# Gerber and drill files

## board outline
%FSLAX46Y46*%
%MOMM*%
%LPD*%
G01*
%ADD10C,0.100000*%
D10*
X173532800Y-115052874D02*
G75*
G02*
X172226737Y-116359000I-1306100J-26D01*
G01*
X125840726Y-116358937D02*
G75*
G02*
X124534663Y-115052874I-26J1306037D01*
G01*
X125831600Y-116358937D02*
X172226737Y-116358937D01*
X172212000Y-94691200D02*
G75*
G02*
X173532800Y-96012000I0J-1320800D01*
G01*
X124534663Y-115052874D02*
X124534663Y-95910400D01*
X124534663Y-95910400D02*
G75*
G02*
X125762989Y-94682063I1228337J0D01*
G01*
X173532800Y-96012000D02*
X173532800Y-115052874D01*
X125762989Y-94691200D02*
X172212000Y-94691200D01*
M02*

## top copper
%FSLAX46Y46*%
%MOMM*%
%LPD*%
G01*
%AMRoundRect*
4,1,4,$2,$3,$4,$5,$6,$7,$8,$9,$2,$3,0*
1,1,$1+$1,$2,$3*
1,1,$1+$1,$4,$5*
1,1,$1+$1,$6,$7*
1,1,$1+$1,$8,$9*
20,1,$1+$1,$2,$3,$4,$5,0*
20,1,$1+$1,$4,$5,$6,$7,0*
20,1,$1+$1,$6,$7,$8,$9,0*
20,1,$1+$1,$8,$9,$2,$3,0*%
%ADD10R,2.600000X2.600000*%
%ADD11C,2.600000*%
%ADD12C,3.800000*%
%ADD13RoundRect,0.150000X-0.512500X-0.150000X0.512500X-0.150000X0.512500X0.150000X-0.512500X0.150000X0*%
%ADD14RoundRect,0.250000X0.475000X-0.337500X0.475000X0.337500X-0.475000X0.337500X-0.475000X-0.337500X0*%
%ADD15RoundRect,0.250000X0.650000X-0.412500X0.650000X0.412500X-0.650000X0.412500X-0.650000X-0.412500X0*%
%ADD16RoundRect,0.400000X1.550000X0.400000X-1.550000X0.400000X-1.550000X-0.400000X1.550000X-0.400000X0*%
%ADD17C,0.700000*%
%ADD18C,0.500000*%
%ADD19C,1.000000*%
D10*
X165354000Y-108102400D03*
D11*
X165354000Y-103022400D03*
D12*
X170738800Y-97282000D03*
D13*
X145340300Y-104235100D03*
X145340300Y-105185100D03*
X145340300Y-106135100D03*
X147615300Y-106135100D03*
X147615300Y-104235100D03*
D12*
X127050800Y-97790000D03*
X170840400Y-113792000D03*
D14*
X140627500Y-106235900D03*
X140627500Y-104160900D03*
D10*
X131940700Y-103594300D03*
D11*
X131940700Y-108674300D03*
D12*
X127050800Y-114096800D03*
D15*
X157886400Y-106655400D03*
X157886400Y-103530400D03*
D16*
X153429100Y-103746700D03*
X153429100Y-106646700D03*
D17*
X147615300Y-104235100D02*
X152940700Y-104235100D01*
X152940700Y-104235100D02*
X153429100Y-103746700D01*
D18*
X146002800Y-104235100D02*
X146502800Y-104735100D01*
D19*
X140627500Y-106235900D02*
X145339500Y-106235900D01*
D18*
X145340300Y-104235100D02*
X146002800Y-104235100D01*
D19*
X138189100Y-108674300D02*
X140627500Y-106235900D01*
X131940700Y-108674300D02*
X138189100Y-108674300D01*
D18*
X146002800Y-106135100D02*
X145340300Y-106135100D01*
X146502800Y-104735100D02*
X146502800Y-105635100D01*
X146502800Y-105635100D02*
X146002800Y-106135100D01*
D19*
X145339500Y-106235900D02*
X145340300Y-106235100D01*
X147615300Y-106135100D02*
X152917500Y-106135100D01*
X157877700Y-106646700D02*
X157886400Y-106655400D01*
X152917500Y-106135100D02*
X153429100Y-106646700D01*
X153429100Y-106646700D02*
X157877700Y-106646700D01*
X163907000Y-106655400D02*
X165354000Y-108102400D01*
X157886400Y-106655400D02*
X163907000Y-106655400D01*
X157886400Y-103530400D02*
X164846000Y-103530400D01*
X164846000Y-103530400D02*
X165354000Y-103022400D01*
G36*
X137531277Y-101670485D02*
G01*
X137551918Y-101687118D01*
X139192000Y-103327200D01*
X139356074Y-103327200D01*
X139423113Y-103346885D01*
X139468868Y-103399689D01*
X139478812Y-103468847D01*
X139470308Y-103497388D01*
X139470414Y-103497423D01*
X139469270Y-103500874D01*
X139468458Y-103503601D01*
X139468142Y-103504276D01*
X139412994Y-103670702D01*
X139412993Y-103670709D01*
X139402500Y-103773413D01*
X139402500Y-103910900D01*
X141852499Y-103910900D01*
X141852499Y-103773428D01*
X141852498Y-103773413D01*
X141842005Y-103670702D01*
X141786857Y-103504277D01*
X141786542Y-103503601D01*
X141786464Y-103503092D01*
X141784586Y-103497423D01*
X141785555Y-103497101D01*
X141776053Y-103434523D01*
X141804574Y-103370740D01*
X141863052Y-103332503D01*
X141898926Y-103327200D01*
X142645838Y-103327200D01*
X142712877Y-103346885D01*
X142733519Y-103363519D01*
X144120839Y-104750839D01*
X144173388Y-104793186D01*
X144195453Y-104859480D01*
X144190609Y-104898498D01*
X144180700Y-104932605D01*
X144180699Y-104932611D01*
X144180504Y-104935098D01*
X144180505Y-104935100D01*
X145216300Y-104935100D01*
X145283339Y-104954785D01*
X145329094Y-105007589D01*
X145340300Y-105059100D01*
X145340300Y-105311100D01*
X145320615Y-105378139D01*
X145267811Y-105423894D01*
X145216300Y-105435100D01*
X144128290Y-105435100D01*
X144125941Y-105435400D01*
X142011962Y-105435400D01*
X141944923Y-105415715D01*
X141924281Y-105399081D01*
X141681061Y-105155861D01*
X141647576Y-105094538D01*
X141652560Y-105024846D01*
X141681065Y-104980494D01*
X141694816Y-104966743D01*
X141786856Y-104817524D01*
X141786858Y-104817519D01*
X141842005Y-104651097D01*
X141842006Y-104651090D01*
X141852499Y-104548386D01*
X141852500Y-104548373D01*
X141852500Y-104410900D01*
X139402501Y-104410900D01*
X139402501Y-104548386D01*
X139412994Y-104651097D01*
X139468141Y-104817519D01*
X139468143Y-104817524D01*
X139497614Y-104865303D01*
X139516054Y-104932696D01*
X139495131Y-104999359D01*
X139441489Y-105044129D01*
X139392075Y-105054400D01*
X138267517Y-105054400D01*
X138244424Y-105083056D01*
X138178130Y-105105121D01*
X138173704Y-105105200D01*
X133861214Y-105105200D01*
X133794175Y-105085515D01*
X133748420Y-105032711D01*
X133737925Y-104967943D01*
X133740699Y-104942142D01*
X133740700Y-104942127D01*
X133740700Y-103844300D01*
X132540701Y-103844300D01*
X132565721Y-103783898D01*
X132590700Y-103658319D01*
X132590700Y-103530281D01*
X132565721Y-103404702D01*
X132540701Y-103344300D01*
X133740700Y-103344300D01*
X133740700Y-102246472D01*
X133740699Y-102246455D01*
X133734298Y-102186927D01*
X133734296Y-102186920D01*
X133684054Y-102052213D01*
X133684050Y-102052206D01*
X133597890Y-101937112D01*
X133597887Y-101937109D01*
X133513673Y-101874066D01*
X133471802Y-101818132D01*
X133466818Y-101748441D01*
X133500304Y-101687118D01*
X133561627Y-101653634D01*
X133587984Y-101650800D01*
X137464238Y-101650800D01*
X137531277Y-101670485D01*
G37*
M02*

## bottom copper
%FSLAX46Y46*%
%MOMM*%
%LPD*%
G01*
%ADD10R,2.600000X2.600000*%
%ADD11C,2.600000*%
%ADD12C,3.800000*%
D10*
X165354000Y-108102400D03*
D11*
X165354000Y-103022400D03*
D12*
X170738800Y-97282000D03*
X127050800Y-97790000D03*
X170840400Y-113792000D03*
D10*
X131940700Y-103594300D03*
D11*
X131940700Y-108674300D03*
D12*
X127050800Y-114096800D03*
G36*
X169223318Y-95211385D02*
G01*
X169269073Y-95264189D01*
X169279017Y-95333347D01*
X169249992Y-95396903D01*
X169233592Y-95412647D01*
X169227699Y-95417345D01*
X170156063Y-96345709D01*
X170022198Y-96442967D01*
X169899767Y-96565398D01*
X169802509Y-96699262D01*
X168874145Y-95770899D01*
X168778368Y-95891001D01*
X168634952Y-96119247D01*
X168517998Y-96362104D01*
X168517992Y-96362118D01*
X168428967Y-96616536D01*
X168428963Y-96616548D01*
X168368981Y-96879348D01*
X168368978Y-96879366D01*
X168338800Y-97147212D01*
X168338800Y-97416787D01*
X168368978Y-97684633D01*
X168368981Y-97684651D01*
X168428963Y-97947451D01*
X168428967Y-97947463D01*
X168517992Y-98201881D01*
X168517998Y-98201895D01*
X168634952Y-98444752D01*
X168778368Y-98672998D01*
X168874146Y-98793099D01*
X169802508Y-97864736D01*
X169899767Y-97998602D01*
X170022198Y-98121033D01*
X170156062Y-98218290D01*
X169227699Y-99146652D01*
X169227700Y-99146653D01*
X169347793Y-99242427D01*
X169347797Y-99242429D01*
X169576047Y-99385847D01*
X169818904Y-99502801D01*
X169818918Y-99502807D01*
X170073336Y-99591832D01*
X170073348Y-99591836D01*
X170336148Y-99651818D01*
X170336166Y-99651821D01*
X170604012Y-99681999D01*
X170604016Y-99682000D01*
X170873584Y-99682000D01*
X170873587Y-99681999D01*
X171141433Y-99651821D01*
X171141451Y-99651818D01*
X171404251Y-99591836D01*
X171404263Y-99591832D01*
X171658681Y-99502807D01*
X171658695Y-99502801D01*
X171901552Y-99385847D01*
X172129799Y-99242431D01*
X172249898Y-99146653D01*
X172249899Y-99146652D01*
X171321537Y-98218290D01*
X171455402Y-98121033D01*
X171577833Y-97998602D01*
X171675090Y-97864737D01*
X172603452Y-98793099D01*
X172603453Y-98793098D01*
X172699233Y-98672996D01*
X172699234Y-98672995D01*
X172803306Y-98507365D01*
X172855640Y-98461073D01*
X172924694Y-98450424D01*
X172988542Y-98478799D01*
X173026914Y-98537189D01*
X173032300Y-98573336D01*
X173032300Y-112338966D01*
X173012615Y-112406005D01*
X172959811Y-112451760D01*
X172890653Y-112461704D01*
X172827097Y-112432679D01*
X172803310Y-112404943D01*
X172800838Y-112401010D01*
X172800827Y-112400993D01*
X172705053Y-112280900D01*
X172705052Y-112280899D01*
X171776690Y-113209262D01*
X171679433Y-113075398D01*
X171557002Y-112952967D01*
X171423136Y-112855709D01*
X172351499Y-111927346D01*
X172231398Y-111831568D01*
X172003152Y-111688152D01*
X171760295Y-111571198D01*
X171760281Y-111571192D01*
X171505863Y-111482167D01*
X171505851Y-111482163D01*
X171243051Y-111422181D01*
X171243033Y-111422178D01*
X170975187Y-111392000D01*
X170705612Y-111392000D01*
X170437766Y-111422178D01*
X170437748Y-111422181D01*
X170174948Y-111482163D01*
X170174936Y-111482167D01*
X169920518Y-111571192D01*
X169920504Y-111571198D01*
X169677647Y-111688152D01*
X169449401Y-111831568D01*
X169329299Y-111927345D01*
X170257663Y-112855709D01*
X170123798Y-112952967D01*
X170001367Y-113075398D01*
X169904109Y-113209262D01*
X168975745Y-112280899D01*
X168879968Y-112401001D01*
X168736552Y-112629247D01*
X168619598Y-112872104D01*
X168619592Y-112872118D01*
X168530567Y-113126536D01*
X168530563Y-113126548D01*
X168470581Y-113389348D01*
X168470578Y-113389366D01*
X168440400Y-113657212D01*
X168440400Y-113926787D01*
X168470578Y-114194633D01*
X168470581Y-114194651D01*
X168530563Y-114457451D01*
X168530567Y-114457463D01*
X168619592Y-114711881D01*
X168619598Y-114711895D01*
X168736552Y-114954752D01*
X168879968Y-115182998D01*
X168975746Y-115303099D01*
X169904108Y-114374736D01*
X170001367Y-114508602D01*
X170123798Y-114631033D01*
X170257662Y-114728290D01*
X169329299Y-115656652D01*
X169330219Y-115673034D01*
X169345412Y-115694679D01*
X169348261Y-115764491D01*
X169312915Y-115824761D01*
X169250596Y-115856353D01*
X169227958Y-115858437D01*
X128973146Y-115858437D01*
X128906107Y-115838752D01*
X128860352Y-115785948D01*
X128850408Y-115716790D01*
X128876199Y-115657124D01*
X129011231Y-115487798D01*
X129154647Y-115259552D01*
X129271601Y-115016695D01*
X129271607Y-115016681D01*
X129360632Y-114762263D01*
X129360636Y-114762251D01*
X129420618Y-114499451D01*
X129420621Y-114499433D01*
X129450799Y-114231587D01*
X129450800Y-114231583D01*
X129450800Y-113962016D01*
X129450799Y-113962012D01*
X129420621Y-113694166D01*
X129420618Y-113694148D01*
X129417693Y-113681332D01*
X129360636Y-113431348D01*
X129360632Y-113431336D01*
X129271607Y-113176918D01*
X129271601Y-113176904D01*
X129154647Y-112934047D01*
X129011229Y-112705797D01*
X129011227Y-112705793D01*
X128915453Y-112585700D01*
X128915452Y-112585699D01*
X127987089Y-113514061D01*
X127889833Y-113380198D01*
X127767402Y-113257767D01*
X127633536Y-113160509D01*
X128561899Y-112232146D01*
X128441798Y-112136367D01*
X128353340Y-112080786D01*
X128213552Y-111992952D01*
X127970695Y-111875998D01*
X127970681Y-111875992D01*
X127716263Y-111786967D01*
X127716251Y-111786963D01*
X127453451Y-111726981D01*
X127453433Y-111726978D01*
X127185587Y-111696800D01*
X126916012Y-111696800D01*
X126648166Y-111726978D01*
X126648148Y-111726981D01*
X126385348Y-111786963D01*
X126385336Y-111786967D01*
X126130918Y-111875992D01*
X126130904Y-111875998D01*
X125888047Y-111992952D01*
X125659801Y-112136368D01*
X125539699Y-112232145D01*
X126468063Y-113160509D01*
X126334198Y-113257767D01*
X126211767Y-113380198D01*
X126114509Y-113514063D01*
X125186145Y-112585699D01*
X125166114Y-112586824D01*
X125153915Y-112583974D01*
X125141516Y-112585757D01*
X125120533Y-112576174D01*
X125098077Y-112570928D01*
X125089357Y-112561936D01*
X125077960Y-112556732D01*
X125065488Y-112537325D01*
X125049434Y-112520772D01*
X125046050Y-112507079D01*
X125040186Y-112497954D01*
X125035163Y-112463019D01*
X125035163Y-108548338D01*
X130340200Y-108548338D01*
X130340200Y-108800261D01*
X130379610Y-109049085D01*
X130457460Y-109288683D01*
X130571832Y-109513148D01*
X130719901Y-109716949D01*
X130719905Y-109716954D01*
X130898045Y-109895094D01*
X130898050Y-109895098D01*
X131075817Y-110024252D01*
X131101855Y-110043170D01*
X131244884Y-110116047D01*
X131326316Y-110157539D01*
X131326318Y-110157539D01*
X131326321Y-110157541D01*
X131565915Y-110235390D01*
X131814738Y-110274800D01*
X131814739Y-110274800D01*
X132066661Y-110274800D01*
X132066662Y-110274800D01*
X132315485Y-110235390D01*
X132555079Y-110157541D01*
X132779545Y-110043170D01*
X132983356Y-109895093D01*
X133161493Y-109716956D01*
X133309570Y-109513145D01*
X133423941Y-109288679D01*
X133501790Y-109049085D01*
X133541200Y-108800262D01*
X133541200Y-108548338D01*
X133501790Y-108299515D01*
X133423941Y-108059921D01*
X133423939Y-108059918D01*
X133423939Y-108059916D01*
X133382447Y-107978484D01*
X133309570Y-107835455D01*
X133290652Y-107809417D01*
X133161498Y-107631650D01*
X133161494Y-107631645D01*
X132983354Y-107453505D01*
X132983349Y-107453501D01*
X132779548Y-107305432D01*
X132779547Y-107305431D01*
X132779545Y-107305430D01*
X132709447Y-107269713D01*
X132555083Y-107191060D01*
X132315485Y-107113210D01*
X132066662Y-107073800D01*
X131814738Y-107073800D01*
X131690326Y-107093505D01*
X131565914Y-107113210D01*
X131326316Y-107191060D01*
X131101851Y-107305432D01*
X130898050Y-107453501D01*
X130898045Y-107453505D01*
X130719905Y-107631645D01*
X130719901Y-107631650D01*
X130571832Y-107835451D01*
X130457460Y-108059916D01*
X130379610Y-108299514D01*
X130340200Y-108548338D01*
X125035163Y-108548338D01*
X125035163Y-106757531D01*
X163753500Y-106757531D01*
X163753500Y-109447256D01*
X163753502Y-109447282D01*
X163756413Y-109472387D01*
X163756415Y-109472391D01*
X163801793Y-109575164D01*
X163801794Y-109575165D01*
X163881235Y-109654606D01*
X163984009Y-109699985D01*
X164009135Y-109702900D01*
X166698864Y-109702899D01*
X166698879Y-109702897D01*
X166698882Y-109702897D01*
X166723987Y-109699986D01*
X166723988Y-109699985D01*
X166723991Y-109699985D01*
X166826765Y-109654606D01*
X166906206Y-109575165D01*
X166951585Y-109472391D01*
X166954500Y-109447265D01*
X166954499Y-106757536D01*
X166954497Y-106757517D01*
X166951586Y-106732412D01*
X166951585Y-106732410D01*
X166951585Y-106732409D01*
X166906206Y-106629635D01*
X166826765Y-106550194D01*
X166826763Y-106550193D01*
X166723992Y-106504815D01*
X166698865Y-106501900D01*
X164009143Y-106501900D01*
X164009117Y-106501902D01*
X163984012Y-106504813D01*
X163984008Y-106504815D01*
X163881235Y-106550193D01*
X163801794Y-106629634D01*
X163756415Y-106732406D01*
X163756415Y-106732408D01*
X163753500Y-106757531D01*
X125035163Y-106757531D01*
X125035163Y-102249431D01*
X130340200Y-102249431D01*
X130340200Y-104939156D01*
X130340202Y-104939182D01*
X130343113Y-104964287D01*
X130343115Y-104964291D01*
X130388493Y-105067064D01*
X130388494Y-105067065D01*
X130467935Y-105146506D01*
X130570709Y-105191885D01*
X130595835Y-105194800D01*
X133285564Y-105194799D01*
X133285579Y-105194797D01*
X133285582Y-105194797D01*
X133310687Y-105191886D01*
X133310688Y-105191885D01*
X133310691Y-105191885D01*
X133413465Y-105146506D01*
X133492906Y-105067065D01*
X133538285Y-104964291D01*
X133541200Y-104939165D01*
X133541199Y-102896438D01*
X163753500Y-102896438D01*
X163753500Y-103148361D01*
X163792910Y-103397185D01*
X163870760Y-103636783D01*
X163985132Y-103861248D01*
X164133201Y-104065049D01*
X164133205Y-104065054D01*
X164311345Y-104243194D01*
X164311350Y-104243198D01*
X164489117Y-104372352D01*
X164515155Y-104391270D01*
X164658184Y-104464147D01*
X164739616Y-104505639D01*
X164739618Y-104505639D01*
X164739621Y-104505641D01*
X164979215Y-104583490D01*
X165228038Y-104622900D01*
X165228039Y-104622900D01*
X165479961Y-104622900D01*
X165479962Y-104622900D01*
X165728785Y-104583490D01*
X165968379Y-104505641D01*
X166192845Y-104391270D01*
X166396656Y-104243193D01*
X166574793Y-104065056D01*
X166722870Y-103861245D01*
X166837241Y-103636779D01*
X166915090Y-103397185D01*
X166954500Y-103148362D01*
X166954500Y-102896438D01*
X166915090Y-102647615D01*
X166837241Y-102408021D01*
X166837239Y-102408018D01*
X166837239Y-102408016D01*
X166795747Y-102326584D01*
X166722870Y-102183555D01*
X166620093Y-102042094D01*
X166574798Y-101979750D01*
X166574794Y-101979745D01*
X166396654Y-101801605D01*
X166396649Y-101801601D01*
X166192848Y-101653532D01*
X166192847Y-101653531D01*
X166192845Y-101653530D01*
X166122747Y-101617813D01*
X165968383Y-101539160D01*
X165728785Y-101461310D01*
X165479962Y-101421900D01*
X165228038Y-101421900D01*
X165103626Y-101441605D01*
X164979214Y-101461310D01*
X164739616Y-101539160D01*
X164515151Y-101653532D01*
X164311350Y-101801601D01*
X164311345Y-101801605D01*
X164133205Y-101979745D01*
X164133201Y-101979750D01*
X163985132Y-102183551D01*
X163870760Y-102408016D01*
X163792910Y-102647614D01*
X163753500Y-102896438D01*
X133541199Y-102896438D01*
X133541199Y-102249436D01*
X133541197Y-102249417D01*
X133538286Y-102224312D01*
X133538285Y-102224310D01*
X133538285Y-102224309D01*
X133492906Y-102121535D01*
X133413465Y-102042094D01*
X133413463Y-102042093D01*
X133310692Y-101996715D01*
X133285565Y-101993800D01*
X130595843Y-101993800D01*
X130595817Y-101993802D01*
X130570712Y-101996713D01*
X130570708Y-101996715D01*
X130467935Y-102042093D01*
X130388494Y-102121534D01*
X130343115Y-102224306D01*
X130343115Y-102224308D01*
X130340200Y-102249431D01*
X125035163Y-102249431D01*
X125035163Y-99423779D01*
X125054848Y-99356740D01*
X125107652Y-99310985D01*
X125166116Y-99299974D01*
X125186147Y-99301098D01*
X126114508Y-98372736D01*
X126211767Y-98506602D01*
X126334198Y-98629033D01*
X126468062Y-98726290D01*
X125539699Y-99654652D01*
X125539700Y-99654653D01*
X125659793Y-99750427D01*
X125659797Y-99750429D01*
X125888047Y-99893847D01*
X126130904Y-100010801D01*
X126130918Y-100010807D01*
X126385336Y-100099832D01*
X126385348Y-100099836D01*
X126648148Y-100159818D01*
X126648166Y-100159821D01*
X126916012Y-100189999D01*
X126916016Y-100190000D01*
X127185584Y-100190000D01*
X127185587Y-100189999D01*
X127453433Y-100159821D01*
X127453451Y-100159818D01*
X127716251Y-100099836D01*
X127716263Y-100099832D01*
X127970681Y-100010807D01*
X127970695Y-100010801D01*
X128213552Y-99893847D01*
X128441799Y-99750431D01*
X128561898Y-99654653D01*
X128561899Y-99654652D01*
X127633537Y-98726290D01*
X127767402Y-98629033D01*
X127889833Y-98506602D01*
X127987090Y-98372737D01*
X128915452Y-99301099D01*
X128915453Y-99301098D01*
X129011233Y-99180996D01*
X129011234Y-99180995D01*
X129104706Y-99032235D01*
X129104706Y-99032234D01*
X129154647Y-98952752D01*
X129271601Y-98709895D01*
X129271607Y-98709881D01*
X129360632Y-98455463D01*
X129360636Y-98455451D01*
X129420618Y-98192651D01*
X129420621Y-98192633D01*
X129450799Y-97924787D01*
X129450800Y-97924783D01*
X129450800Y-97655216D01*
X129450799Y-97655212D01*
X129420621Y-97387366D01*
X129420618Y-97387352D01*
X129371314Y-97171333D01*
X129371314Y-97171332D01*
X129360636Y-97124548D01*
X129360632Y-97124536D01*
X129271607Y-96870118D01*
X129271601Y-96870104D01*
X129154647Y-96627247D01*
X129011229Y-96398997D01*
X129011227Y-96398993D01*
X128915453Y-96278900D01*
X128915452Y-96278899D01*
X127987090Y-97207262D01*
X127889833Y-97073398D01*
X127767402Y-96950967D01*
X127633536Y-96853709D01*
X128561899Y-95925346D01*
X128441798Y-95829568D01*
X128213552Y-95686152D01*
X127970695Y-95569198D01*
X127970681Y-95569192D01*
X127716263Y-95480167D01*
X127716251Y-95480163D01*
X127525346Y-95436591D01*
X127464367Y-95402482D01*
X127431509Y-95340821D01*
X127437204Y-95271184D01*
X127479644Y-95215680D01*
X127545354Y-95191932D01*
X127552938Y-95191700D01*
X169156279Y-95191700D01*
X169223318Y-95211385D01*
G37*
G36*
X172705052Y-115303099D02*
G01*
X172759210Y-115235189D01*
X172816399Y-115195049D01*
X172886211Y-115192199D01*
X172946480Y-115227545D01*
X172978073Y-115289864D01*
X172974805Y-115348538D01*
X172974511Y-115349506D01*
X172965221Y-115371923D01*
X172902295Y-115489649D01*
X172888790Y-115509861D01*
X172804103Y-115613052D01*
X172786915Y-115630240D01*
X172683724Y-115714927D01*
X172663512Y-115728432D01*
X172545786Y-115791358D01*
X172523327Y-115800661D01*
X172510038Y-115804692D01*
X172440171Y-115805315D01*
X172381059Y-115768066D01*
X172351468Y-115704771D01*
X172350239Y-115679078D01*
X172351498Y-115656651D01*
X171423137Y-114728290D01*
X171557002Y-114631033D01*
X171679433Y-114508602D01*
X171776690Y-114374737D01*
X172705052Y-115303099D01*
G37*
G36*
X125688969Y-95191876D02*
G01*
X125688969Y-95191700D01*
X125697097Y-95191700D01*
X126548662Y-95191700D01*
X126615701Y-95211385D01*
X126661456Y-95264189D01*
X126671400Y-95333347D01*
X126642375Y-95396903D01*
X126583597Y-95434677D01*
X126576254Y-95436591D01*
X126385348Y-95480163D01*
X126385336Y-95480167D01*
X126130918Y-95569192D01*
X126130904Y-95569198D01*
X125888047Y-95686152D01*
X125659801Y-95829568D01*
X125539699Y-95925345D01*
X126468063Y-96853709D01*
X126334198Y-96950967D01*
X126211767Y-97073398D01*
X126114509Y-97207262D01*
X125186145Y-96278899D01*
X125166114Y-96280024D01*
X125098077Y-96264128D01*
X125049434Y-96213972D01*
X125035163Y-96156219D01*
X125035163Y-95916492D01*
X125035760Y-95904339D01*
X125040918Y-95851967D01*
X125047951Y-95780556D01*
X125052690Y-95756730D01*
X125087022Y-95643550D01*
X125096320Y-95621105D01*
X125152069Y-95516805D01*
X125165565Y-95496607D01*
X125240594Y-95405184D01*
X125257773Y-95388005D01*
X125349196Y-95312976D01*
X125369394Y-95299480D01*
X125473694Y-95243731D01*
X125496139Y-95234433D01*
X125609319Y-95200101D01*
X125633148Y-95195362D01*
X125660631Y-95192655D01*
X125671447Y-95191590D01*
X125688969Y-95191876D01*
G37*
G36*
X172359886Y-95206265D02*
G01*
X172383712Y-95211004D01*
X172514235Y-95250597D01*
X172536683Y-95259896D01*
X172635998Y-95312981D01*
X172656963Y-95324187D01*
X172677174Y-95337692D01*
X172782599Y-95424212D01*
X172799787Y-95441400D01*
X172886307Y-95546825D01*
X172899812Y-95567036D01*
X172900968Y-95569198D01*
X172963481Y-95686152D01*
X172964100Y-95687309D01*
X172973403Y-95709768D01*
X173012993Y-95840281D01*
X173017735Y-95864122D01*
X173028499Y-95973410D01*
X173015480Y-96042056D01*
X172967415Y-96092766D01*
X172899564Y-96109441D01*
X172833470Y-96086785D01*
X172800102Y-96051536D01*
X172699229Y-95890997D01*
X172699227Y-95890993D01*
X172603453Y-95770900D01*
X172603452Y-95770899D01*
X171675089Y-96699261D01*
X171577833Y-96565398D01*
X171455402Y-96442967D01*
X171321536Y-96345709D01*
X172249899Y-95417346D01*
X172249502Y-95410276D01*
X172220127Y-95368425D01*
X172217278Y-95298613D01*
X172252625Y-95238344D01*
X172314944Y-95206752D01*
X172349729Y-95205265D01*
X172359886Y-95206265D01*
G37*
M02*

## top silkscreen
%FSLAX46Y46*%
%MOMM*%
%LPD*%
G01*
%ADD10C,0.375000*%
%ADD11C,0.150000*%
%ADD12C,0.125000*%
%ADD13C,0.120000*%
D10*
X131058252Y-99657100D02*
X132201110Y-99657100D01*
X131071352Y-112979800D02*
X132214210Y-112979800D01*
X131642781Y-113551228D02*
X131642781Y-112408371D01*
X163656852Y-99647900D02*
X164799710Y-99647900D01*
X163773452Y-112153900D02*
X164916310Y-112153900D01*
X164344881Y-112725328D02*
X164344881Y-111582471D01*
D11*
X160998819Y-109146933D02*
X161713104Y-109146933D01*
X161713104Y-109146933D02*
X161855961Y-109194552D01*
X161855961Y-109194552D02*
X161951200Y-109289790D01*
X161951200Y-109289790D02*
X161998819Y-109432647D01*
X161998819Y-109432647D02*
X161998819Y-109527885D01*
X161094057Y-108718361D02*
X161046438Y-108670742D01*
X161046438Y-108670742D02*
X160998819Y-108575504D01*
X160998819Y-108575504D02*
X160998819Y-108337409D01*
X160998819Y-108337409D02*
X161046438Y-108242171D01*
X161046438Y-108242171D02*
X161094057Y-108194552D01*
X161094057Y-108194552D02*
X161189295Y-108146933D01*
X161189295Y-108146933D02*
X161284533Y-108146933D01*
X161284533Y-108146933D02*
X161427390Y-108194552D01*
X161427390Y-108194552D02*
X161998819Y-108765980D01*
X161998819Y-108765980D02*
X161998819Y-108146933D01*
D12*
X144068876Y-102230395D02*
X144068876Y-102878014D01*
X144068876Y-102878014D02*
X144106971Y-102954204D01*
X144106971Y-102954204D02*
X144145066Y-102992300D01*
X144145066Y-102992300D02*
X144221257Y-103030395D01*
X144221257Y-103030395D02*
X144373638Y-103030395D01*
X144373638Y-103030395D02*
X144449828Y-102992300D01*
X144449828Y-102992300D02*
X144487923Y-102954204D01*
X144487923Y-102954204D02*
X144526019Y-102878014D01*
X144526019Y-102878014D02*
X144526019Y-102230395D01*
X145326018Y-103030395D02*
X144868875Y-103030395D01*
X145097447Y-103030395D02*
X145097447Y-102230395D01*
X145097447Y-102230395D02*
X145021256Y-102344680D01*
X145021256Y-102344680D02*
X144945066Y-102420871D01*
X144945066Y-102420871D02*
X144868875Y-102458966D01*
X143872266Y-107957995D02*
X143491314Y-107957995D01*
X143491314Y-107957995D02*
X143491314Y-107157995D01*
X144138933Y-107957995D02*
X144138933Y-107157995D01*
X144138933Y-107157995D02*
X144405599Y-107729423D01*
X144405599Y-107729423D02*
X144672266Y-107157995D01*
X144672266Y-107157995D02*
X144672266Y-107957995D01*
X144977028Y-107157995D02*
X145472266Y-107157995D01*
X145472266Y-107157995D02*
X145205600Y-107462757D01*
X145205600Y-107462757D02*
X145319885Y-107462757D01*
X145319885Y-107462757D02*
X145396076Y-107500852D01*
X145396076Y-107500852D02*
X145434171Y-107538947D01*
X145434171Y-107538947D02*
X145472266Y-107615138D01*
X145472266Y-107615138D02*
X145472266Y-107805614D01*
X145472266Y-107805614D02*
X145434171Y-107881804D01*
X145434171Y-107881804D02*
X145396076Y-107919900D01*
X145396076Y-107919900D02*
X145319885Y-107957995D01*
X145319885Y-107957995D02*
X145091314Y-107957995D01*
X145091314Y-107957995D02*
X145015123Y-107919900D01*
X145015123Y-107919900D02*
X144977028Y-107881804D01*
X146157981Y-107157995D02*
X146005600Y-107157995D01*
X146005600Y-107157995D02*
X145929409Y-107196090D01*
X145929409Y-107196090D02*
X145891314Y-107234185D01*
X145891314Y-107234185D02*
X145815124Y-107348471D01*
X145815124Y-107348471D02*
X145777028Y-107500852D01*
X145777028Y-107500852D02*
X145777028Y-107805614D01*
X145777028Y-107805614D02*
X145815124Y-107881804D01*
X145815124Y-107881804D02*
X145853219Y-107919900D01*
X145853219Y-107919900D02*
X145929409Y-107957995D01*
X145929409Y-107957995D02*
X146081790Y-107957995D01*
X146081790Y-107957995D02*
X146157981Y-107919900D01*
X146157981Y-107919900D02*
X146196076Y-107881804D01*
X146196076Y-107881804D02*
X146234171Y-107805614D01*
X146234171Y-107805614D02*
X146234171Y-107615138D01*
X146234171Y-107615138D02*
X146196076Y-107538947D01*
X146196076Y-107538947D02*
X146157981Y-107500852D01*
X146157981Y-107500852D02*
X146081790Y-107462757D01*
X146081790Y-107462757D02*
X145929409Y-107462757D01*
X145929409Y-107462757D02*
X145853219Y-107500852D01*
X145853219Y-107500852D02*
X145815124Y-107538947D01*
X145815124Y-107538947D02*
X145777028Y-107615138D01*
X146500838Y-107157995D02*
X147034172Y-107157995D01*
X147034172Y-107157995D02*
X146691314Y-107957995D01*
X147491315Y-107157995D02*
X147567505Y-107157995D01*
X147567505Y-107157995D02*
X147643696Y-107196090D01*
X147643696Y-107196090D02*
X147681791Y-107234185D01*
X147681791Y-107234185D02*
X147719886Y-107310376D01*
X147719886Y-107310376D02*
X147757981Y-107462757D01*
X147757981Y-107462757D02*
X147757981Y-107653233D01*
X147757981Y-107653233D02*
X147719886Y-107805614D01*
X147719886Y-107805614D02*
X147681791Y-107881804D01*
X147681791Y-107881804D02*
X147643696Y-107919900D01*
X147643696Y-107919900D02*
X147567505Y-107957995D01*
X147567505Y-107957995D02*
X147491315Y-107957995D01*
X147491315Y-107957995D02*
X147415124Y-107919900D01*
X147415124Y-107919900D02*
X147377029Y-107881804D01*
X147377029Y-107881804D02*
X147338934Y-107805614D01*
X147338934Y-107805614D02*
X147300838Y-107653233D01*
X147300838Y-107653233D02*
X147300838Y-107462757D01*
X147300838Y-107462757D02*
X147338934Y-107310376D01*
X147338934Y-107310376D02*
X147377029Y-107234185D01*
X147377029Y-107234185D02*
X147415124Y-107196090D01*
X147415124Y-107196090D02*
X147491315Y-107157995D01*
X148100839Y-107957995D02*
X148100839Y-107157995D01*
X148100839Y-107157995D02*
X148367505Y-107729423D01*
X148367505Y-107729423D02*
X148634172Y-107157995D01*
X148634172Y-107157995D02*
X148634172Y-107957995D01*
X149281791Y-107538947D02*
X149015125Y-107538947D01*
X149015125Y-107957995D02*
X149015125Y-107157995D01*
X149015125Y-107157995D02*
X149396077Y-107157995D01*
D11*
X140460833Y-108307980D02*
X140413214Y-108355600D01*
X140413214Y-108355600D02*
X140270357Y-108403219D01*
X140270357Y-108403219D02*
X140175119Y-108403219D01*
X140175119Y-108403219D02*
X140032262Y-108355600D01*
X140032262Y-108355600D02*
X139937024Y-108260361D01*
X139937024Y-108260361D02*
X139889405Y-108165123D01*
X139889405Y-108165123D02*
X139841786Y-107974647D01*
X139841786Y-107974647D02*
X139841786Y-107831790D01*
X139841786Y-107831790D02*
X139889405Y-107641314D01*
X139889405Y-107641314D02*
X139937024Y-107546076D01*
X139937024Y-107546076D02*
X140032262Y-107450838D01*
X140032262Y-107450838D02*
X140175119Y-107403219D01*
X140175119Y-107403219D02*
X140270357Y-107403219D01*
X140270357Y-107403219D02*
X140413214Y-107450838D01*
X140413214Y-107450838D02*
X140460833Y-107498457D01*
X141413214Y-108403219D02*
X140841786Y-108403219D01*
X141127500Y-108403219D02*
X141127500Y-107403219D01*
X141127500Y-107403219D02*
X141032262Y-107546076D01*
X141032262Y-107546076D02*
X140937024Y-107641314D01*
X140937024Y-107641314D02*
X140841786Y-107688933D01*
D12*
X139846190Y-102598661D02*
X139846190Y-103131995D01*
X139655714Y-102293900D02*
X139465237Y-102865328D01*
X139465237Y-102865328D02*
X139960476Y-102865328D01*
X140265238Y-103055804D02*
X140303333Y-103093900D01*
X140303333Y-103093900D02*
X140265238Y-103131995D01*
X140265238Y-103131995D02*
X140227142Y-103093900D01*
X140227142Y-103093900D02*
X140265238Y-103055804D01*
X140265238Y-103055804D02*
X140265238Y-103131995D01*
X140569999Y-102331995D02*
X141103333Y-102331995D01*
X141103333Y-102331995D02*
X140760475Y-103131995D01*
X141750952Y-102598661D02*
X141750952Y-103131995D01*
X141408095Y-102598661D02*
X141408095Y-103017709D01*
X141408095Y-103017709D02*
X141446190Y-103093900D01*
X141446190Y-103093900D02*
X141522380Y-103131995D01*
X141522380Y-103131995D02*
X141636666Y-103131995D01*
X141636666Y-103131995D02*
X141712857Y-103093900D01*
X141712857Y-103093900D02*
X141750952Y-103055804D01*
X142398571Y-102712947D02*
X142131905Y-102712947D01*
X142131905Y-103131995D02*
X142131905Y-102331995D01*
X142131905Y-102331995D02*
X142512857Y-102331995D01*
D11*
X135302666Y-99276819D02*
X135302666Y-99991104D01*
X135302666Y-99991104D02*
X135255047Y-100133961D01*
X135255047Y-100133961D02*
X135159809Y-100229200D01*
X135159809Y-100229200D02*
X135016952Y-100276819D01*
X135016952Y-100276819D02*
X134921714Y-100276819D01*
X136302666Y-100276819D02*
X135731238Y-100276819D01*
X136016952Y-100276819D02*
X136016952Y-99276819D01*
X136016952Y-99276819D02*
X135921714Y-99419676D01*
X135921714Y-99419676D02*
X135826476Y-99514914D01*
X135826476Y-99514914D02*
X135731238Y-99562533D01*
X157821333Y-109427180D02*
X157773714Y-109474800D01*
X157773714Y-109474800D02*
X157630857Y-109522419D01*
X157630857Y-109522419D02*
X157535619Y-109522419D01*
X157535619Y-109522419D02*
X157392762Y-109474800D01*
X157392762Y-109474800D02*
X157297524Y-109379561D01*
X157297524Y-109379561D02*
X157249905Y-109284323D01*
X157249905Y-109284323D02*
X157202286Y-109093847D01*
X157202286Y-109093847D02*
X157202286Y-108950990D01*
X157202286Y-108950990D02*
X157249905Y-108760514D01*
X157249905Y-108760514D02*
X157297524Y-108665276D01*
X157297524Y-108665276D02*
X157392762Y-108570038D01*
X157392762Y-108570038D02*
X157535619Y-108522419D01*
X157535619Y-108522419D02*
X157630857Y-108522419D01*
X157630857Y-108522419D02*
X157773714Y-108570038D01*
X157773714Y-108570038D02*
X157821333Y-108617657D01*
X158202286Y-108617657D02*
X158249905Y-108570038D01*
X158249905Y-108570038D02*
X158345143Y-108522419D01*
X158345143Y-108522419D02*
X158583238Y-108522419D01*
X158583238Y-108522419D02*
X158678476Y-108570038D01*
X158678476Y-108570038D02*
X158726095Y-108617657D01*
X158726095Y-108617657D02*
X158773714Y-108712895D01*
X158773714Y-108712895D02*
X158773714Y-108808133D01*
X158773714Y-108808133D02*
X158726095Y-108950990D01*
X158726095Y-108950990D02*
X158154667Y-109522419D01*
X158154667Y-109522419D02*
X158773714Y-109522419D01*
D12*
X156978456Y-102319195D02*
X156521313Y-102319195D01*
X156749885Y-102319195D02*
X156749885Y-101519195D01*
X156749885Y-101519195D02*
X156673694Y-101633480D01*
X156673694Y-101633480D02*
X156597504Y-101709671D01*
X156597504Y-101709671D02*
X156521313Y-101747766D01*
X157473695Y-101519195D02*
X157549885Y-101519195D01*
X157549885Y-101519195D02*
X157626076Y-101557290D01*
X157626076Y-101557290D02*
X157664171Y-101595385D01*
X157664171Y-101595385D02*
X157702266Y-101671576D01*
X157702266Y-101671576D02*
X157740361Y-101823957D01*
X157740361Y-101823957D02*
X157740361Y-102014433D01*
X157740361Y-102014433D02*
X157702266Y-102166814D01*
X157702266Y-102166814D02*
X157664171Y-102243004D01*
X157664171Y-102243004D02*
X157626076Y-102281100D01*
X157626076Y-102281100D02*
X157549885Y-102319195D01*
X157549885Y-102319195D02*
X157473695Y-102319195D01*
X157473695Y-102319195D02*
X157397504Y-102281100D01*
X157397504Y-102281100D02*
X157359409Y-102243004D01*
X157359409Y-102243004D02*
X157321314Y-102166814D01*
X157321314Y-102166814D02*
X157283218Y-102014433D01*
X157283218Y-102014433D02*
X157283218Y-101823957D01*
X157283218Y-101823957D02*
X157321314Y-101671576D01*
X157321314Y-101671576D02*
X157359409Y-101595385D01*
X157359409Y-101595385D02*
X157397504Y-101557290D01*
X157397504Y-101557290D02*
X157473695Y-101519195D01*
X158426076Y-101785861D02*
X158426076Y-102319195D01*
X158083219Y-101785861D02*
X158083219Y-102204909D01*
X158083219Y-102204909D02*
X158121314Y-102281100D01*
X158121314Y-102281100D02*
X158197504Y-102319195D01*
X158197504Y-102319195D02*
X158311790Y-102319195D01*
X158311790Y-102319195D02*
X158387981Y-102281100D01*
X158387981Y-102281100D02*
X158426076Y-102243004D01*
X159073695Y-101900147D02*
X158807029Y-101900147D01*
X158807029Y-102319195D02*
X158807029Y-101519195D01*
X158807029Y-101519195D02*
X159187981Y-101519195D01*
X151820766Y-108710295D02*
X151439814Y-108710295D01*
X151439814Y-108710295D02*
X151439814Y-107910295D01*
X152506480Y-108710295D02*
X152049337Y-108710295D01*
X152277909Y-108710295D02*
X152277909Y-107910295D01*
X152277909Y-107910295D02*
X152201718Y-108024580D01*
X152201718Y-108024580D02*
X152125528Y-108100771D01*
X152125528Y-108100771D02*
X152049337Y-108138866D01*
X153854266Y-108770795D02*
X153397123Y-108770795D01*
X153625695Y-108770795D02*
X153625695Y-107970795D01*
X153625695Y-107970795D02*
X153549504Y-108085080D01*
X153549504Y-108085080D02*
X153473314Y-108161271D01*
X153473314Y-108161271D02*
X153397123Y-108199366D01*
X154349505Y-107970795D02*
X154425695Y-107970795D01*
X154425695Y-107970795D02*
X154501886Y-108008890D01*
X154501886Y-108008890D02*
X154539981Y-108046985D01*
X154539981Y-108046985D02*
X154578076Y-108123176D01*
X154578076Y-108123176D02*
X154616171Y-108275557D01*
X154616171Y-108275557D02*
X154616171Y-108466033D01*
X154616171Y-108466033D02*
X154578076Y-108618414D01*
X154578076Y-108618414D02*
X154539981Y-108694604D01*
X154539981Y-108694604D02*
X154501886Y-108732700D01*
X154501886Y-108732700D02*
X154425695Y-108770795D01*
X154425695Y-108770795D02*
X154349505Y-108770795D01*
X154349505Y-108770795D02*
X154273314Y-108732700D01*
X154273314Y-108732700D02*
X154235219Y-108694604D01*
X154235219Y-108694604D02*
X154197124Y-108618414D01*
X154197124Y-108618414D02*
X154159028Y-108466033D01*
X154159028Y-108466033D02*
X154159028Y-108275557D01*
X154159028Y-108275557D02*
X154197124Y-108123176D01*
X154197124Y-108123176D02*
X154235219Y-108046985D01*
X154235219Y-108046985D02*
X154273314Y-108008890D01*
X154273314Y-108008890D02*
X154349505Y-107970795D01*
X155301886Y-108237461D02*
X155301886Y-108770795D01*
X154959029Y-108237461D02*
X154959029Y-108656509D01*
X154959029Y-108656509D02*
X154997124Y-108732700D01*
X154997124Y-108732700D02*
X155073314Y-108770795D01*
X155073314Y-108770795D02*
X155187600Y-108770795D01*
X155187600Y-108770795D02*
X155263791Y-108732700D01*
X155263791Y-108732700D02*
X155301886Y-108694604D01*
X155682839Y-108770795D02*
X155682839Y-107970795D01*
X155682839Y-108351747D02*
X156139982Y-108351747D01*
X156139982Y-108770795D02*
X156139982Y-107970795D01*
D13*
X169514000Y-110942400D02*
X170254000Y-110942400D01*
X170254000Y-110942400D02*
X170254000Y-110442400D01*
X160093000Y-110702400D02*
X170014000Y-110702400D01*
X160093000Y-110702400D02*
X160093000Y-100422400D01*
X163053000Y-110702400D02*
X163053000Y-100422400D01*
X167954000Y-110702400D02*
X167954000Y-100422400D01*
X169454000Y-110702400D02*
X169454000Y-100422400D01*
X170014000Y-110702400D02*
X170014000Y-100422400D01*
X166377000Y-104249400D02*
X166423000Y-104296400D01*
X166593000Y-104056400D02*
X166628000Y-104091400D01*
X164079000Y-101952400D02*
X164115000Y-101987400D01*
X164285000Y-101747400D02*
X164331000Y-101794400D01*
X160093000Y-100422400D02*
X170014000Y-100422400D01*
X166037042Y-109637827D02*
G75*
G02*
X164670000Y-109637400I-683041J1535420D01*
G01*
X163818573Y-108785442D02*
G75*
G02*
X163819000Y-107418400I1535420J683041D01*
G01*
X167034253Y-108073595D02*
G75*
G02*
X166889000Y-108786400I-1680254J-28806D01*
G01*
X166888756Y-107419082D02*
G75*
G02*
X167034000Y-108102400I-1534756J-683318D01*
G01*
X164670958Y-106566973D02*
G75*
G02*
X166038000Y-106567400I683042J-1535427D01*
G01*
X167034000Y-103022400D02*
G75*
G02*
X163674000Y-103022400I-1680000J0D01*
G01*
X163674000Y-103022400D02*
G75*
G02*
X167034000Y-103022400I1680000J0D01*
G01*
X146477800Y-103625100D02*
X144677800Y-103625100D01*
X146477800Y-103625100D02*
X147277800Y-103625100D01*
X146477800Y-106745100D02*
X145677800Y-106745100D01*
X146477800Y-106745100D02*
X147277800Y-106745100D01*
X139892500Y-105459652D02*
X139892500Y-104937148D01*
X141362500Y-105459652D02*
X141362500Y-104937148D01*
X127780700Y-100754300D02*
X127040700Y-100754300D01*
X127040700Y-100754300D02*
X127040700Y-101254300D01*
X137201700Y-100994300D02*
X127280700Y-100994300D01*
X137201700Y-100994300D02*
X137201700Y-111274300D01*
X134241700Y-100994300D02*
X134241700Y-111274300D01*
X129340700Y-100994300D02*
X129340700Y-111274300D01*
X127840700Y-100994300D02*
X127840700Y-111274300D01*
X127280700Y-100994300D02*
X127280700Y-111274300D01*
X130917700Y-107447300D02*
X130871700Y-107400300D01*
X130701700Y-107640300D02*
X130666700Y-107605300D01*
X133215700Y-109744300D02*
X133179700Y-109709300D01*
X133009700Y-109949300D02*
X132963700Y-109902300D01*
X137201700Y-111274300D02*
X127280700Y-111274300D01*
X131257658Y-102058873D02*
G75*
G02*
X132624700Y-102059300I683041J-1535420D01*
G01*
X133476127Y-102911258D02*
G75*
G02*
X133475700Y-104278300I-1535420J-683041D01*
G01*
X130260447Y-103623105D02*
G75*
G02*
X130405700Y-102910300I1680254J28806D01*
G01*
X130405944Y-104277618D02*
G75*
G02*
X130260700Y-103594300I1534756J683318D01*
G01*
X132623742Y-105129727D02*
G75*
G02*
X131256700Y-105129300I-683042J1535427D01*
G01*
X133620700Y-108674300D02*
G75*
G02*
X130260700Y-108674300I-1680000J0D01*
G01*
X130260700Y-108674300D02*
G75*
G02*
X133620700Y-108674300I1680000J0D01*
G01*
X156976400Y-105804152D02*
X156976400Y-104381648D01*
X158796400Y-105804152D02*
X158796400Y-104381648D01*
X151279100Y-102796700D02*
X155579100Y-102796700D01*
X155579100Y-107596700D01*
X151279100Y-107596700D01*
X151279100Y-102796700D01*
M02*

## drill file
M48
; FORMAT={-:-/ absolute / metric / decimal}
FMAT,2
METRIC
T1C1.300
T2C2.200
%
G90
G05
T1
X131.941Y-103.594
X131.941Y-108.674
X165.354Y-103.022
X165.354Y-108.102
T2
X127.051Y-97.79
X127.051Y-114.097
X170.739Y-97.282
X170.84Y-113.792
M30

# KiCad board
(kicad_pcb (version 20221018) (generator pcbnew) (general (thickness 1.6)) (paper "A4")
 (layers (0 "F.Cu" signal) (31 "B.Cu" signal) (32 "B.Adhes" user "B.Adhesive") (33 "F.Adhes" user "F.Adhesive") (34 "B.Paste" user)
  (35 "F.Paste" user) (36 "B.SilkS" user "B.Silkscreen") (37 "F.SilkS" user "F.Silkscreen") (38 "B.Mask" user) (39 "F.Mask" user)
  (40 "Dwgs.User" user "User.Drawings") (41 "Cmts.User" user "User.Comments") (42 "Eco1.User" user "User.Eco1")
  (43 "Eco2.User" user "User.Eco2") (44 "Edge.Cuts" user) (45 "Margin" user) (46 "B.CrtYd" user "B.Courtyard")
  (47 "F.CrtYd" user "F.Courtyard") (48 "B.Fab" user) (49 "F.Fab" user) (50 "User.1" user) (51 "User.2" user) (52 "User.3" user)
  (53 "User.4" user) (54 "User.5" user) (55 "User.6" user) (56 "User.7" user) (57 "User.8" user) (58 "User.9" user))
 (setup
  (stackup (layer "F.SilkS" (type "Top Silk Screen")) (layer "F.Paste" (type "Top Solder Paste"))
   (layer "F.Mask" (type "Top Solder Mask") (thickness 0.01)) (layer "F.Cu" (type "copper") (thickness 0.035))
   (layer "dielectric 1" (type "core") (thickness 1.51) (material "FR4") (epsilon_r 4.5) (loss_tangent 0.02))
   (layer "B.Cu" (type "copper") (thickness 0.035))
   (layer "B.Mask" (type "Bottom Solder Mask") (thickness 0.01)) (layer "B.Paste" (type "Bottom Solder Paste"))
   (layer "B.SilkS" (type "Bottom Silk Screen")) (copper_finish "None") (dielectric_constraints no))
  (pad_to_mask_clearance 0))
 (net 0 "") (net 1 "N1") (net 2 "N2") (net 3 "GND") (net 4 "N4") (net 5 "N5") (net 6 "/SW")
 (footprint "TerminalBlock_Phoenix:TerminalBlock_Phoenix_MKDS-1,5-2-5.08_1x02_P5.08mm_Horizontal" (layer "F.Cu") (at 165.354 108.1024 90)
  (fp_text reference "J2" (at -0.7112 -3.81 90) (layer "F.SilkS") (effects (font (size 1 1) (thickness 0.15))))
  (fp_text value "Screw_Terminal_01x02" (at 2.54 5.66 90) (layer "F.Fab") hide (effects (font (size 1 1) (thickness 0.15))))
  (fp_line (start -2.84 4.16) (end -2.84 4.9) (stroke (width 0.12) (type solid)) (layer "F.SilkS"))
  (fp_line (start -2.84 4.9) (end -2.34 4.9) (stroke (width 0.12) (type solid)) (layer "F.SilkS"))
  (fp_line (start -2.6 -5.261) (end -2.6 4.66) (stroke (width 0.12) (type solid)) (layer "F.SilkS"))
  (fp_line (start -2.6 -5.261) (end 7.68 -5.261) (stroke (width 0.12) (type solid)) (layer "F.SilkS"))
  (fp_line (start -2.6 -2.301) (end 7.68 -2.301) (stroke (width 0.12) (type solid)) (layer "F.SilkS"))
  (fp_line (start -2.6 2.6) (end 7.68 2.6) (stroke (width 0.12) (type solid)) (layer "F.SilkS"))
  (fp_line (start -2.6 4.1) (end 7.68 4.1) (stroke (width 0.12) (type solid)) (layer "F.SilkS"))
  (fp_line (start -2.6 4.66) (end 7.68 4.66) (stroke (width 0.12) (type solid)) (layer "F.SilkS"))
  (fp_line (start 3.853 1.023) (end 3.806 1.069) (stroke (width 0.12) (type solid)) (layer "F.SilkS"))
  (fp_line (start 4.046 1.239) (end 4.011 1.274) (stroke (width 0.12) (type solid)) (layer "F.SilkS"))
  (fp_line (start 6.15 -1.275) (end 6.115 -1.239) (stroke (width 0.12) (type solid)) (layer "F.SilkS"))
  (fp_line (start 6.355 -1.069) (end 6.308 -1.023) (stroke (width 0.12) (type solid)) (layer "F.SilkS"))
  (fp_line (start 7.68 -5.261) (end 7.68 4.66) (stroke (width 0.12) (type solid)) (layer "F.SilkS"))
  (fp_arc (start -1.535427 0.683042) (mid -1.680501 -0.000524) (end -1.535 -0.684) (stroke (width 0.12) (type solid)) (layer "F.SilkS"))
  (fp_arc (start -0.683042 -1.535427) (mid 0.000524 -1.680501) (end 0.684 -1.535) (stroke (width 0.12) (type solid)) (layer "F.SilkS"))
  (fp_arc (start 0.028805 1.680253) (mid -0.335551 1.646659) (end -0.684 1.535) (stroke (width 0.12) (type solid)) (layer "F.SilkS"))
  (fp_arc (start 0.683318 1.534756) (mid 0.349292 1.643288) (end 0 1.68) (stroke (width 0.12) (type solid)) (layer "F.SilkS"))
  (fp_arc (start 1.535427 -0.683042) (mid 1.680501 0.000524) (end 1.535 0.684) (stroke (width 0.12) (type solid)) (layer "F.SilkS"))
  (fp_circle (center 5.08 0) (end 6.76 0) (stroke (width 0.12) (type solid)) (fill none) (layer "F.SilkS"))
  (pad "1" thru_hole rect (at 0 0 90) (size 2.6 2.6) (drill 1.3) (layers "*.Cu" "*.Mask") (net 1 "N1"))
  (pad "2" thru_hole circle (at 5.08 0 90) (size 2.6 2.6) (drill 1.3) (layers "*.Cu" "*.Mask") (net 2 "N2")))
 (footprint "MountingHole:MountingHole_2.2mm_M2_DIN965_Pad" (layer "F.Cu") (at 170.7388 97.282)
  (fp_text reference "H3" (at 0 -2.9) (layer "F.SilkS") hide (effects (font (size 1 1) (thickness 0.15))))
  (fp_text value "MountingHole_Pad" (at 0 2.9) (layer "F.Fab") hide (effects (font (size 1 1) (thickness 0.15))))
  (pad "1" thru_hole circle (at 0 0) (size 3.8 3.8) (drill 2.2) (layers "*.Cu" "*.Mask") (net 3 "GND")))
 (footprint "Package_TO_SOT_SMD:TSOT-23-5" (layer "F.Cu") (at 146.4778 105.1851)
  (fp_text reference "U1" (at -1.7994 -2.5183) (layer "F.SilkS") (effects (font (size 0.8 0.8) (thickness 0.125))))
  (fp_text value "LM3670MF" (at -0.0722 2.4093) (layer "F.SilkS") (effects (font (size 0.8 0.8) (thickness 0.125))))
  (fp_line (start 0 -1.56) (end -1.8 -1.56) (stroke (width 0.12) (type solid)) (layer "F.SilkS"))
  (fp_line (start 0 -1.56) (end 0.8 -1.56) (stroke (width 0.12) (type solid)) (layer "F.SilkS"))
  (fp_line (start 0 1.56) (end -0.8 1.56) (stroke (width 0.12) (type solid)) (layer "F.SilkS"))
  (fp_line (start 0 1.56) (end 0.8 1.56) (stroke (width 0.12) (type solid)) (layer "F.SilkS"))
  (pad "1" smd roundrect (at -1.1375 -0.95) (size 1.325 0.6) (layers "F.Cu" "F.Paste" "F.Mask") (roundrect_rratio 0.25) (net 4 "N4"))
  (pad "2" smd roundrect (at -1.1375 0) (size 1.325 0.6) (layers "F.Cu" "F.Paste" "F.Mask") (roundrect_rratio 0.25) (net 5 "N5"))
  (pad "3" smd roundrect (at -1.1375 0.95) (size 1.325 0.6) (layers "F.Cu" "F.Paste" "F.Mask") (roundrect_rratio 0.25) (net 4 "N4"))
  (pad "4" smd roundrect (at 1.1375 0.95) (size 1.325 0.6) (layers "F.Cu" "F.Paste" "F.Mask") (roundrect_rratio 0.25) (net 1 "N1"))
  (pad "5" smd roundrect (at 1.1375 -0.95) (size 1.325 0.6) (layers "F.Cu" "F.Paste" "F.Mask") (roundrect_rratio 0.25) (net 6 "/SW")))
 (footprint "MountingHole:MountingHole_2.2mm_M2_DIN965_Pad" (layer "F.Cu") (at 127.0508 97.79)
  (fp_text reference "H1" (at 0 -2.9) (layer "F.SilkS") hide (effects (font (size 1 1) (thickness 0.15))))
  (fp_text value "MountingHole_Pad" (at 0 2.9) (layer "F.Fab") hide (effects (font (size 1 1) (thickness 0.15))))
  (pad "1" thru_hole circle (at 0 0) (size 3.8 3.8) (drill 2.2) (layers "*.Cu" "*.Mask") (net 3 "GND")))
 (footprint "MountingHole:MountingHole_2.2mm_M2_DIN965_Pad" (layer "F.Cu") (at 170.8404 113.792)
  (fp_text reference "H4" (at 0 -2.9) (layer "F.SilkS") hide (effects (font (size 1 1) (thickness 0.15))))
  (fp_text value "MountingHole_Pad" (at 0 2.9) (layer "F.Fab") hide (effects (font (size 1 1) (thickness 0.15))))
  (pad "1" thru_hole circle (at 0 0) (size 3.8 3.8) (drill 2.2) (layers "*.Cu" "*.Mask") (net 3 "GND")))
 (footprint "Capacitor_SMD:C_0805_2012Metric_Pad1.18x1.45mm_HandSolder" (layer "F.Cu") (at 140.6275 105.1984 90)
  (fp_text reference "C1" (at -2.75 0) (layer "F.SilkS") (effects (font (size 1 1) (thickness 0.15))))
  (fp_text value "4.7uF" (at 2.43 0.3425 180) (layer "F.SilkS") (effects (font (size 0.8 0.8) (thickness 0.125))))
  (fp_line (start -0.261252 -0.735) (end 0.261252 -0.735) (stroke (width 0.12) (type solid)) (layer "F.SilkS"))
  (fp_line (start -0.261252 0.735) (end 0.261252 0.735) (stroke (width 0.12) (type solid)) (layer "F.SilkS"))
  (pad "1" smd roundrect (at -1.0375 0 90) (size 1.175 1.45) (layers "F.Cu" "F.Paste" "F.Mask") (roundrect_rratio 0.2127659574) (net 4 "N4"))
  (pad "2" smd roundrect (at 1.0375 0 90) (size 1.175 1.45) (layers "F.Cu" "F.Paste" "F.Mask") (roundrect_rratio 0.2127659574) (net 5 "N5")))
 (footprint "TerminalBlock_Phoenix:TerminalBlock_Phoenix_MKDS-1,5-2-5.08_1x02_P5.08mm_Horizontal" (layer "F.Cu") (at 131.9407 103.5943 -90)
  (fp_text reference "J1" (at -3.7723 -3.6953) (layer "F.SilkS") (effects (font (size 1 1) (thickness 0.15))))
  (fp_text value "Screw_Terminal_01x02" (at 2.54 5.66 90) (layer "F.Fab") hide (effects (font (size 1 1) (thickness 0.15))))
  (fp_line (start -2.84 4.16) (end -2.84 4.9) (stroke (width 0.12) (type solid)) (layer "F.SilkS"))
  (fp_line (start -2.84 4.9) (end -2.34 4.9) (stroke (width 0.12) (type solid)) (layer "F.SilkS"))
  (fp_line (start -2.6 -5.261) (end -2.6 4.66) (stroke (width 0.12) (type solid)) (layer "F.SilkS"))
  (fp_line (start -2.6 -5.261) (end 7.68 -5.261) (stroke (width 0.12) (type solid)) (layer "F.SilkS"))
  (fp_line (start -2.6 -2.301) (end 7.68 -2.301) (stroke (width 0.12) (type solid)) (layer "F.SilkS"))
  (fp_line (start -2.6 2.6) (end 7.68 2.6) (stroke (width 0.12) (type solid)) (layer "F.SilkS"))
  (fp_line (start -2.6 4.1) (end 7.68 4.1) (stroke (width 0.12) (type solid)) (layer "F.SilkS"))
  (fp_line (start -2.6 4.66) (end 7.68 4.66) (stroke (width 0.12) (type solid)) (layer "F.SilkS"))
  (fp_line (start 3.853 1.023) (end 3.806 1.069) (stroke (width 0.12) (type solid)) (layer "F.SilkS"))
  (fp_line (start 4.046 1.239) (end 4.011 1.274) (stroke (width 0.12) (type solid)) (layer "F.SilkS"))
  (fp_line (start 6.15 -1.275) (end 6.115 -1.239) (stroke (width 0.12) (type solid)) (layer "F.SilkS"))
  (fp_line (start 6.355 -1.069) (end 6.308 -1.023) (stroke (width 0.12) (type solid)) (layer "F.SilkS"))
  (fp_line (start 7.68 -5.261) (end 7.68 4.66) (stroke (width 0.12) (type solid)) (layer "F.SilkS"))
  (fp_arc (start -1.535427 0.683042) (mid -1.680501 -0.000524) (end -1.535 -0.684) (stroke (width 0.12) (type solid)) (layer "F.SilkS"))
  (fp_arc (start -0.683042 -1.535427) (mid 0.000524 -1.680501) (end 0.684 -1.535) (stroke (width 0.12) (type solid)) (layer "F.SilkS"))
  (fp_arc (start 0.028805 1.680253) (mid -0.335551 1.646659) (end -0.684 1.535) (stroke (width 0.12) (type solid)) (layer "F.SilkS"))
  (fp_arc (start 0.683318 1.534756) (mid 0.349292 1.643288) (end 0 1.68) (stroke (width 0.12) (type solid)) (layer "F.SilkS"))
  (fp_arc (start 1.535427 -0.683042) (mid 1.680501 0.000524) (end 1.535 0.684) (stroke (width 0.12) (type solid)) (layer "F.SilkS"))
  (fp_circle (center 5.08 0) (end 6.76 0) (stroke (width 0.12) (type solid)) (fill none) (layer "F.SilkS"))
  (pad "1" thru_hole rect (at 0 0 270) (size 2.6 2.6) (drill 1.3) (layers "*.Cu" "*.Mask") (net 5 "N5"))
  (pad "2" thru_hole circle (at 5.08 0 270) (size 2.6 2.6) (drill 1.3) (layers "*.Cu" "*.Mask") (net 4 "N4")))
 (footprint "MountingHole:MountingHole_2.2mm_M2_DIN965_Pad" (layer "F.Cu") (at 127.0508 114.0968)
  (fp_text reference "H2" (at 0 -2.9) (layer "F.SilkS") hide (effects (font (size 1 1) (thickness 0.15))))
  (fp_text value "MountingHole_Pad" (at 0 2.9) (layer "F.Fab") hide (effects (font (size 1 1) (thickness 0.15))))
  (pad "1" thru_hole circle (at 0 0) (size 3.8 3.8) (drill 2.2) (layers "*.Cu" "*.Mask") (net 3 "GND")))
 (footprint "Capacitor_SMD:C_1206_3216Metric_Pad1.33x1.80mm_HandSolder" (layer "F.Cu") (at 157.8864 105.0929 90)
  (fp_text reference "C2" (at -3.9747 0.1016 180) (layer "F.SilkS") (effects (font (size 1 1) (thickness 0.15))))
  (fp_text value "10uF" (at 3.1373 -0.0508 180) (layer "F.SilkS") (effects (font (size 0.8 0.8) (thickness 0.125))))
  (fp_line (start -0.711252 -0.91) (end 0.711252 -0.91) (stroke (width 0.12) (type solid)) (layer "F.SilkS"))
  (fp_line (start -0.711252 0.91) (end 0.711252 0.91) (stroke (width 0.12) (type solid)) (layer "F.SilkS"))
  (pad "1" smd roundrect (at -1.5625 0 90) (size 1.325 1.8) (layers "F.Cu" "F.Paste" "F.Mask") (roundrect_rratio 0.1886792453) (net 1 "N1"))
  (pad "2" smd roundrect (at 1.5625 0 90) (size 1.325 1.8) (layers "F.Cu" "F.Paste" "F.Mask") (roundrect_rratio 0.1886792453) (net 2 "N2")))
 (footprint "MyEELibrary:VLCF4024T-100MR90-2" (layer "F.Cu") (at 153.4291 105.1967 180)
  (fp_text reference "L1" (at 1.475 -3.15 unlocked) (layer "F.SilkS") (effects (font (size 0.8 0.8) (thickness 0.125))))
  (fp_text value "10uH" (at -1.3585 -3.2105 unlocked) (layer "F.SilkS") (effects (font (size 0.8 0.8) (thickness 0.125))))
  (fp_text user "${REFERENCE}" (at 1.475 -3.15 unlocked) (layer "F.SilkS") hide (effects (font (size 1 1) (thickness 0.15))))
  (fp_rect (start -2.15 -2.4) (end 2.15 2.4) (stroke (width 0.12) (type default)) (fill none) (layer "F.SilkS"))
  (pad "1" smd roundrect (at 0 1.45 180) (size 3.9 1.6) (layers "F.Cu" "F.Paste" "F.Mask") (roundrect_rratio 0.25) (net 6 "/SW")
   (thermal_bridge_angle 45))
  (pad "2" smd roundrect (at 0 -1.45 180) (size 3.9 1.6) (layers "F.Cu" "F.Paste" "F.Mask") (roundrect_rratio 0.25) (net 1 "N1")
   (thermal_bridge_angle 45)))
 (gr_arc (start 173.5328 115.052874) (mid 173.150263 115.9764) (end 172.226737 116.358937) (stroke (width 0.1) (type default))
  (layer "Edge.Cuts"))
 (gr_arc (start 125.840726 116.358937) (mid 124.9172 115.9764) (end 124.534663 115.052874) (stroke (width 0.1) (type default))
  (layer "Edge.Cuts"))
 (gr_line (start 125.8316 116.358937) (end 172.226737 116.358937) (stroke (width 0.1) (type default)) (layer "Edge.Cuts"))
 (gr_arc (start 172.212 94.6912) (mid 173.145947 95.078053) (end 173.5328 96.012) (stroke (width 0.1) (type default)) (layer "Edge.Cuts"))
 (gr_line (start 124.534663 115.052874) (end 124.534663 95.9104) (stroke (width 0.1) (type default)) (layer "Edge.Cuts"))
 (gr_arc (start 124.534663 95.9104) (mid 124.894431 95.041842) (end 125.762989 94.682074) (stroke (width 0.1) (type default))
  (layer "Edge.Cuts"))
 (gr_line (start 173.5328 96.012) (end 173.5328 115.052874) (stroke (width 0.1) (type default)) (layer "Edge.Cuts"))
 (gr_line (start 125.762989 94.6912) (end 172.212 94.6912) (stroke (width 0.1) (type default)) (layer "Edge.Cuts"))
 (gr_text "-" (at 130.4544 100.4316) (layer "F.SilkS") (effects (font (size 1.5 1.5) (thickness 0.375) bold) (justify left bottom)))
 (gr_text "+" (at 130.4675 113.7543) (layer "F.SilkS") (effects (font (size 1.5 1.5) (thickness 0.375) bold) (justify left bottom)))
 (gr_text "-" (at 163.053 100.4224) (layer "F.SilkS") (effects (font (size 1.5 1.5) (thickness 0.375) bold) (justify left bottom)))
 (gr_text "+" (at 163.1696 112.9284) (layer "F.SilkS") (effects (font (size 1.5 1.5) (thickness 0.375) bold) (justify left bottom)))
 (segment (start 147.6153 104.2351) (end 152.9407 104.2351) (width 0.7) (layer "F.Cu") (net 6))
 (segment (start 152.9407 104.2351) (end 153.4291 103.7467) (width 0.7) (layer "F.Cu") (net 6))
 (segment (start 146.0028 104.2351) (end 146.5028 104.7351) (width 0.5) (layer "F.Cu") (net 4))
 (segment (start 140.6275 106.2359) (end 145.3395 106.2359) (width 1) (layer "F.Cu") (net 4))
 (segment (start 145.3403 104.2351) (end 146.0028 104.2351) (width 0.5) (layer "F.Cu") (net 4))
 (segment (start 138.1891 108.6743) (end 140.6275 106.2359) (width 1) (layer "F.Cu") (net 4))
 (segment (start 131.9407 108.6743) (end 138.1891 108.6743) (width 1) (layer "F.Cu") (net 4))
 (segment (start 146.0028 106.1351) (end 145.3403 106.1351) (width 0.5) (layer "F.Cu") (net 4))
 (segment (start 146.5028 104.7351) (end 146.5028 105.6351) (width 0.5) (layer "F.Cu") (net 4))
 (segment (start 146.5028 105.6351) (end 146.0028 106.1351) (width 0.5) (layer "F.Cu") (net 4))
 (segment (start 145.3395 106.2359) (end 145.3403 106.2351) (width 1) (layer "F.Cu") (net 4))
 (segment (start 147.6153 106.1351) (end 152.9175 106.1351) (width 1) (layer "F.Cu") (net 1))
 (segment (start 157.8777 106.6467) (end 157.8864 106.6554) (width 1) (layer "F.Cu") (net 1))
 (segment (start 152.9175 106.1351) (end 153.4291 106.6467) (width 1) (layer "F.Cu") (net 1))
 (segment (start 153.4291 106.6467) (end 157.8777 106.6467) (width 1) (layer "F.Cu") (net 1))
 (segment (start 163.907 106.6554) (end 165.354 108.1024) (width 1) (layer "F.Cu") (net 1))
 (segment (start 157.8864 106.6554) (end 163.907 106.6554) (width 1) (layer "F.Cu") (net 1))
 (segment (start 157.8864 103.5304) (end 164.846 103.5304) (width 1) (layer "F.Cu") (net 2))
 (segment (start 164.846 103.5304) (end 165.354 103.0224) (width 1) (layer "F.Cu") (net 2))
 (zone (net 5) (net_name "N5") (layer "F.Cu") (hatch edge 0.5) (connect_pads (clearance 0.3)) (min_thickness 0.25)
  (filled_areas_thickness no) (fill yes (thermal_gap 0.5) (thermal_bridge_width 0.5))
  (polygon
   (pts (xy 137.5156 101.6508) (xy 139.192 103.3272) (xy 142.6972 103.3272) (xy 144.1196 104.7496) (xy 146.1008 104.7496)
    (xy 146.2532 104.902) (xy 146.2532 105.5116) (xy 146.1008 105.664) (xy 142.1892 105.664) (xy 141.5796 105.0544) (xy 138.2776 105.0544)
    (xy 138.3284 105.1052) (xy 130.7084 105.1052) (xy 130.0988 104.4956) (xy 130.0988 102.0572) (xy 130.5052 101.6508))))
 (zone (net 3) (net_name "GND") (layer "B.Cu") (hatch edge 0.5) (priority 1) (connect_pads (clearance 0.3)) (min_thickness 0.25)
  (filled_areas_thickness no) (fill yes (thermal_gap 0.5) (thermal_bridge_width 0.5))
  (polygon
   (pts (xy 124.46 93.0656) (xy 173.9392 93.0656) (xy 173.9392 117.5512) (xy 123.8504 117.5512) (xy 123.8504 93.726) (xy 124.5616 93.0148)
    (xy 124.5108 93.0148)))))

